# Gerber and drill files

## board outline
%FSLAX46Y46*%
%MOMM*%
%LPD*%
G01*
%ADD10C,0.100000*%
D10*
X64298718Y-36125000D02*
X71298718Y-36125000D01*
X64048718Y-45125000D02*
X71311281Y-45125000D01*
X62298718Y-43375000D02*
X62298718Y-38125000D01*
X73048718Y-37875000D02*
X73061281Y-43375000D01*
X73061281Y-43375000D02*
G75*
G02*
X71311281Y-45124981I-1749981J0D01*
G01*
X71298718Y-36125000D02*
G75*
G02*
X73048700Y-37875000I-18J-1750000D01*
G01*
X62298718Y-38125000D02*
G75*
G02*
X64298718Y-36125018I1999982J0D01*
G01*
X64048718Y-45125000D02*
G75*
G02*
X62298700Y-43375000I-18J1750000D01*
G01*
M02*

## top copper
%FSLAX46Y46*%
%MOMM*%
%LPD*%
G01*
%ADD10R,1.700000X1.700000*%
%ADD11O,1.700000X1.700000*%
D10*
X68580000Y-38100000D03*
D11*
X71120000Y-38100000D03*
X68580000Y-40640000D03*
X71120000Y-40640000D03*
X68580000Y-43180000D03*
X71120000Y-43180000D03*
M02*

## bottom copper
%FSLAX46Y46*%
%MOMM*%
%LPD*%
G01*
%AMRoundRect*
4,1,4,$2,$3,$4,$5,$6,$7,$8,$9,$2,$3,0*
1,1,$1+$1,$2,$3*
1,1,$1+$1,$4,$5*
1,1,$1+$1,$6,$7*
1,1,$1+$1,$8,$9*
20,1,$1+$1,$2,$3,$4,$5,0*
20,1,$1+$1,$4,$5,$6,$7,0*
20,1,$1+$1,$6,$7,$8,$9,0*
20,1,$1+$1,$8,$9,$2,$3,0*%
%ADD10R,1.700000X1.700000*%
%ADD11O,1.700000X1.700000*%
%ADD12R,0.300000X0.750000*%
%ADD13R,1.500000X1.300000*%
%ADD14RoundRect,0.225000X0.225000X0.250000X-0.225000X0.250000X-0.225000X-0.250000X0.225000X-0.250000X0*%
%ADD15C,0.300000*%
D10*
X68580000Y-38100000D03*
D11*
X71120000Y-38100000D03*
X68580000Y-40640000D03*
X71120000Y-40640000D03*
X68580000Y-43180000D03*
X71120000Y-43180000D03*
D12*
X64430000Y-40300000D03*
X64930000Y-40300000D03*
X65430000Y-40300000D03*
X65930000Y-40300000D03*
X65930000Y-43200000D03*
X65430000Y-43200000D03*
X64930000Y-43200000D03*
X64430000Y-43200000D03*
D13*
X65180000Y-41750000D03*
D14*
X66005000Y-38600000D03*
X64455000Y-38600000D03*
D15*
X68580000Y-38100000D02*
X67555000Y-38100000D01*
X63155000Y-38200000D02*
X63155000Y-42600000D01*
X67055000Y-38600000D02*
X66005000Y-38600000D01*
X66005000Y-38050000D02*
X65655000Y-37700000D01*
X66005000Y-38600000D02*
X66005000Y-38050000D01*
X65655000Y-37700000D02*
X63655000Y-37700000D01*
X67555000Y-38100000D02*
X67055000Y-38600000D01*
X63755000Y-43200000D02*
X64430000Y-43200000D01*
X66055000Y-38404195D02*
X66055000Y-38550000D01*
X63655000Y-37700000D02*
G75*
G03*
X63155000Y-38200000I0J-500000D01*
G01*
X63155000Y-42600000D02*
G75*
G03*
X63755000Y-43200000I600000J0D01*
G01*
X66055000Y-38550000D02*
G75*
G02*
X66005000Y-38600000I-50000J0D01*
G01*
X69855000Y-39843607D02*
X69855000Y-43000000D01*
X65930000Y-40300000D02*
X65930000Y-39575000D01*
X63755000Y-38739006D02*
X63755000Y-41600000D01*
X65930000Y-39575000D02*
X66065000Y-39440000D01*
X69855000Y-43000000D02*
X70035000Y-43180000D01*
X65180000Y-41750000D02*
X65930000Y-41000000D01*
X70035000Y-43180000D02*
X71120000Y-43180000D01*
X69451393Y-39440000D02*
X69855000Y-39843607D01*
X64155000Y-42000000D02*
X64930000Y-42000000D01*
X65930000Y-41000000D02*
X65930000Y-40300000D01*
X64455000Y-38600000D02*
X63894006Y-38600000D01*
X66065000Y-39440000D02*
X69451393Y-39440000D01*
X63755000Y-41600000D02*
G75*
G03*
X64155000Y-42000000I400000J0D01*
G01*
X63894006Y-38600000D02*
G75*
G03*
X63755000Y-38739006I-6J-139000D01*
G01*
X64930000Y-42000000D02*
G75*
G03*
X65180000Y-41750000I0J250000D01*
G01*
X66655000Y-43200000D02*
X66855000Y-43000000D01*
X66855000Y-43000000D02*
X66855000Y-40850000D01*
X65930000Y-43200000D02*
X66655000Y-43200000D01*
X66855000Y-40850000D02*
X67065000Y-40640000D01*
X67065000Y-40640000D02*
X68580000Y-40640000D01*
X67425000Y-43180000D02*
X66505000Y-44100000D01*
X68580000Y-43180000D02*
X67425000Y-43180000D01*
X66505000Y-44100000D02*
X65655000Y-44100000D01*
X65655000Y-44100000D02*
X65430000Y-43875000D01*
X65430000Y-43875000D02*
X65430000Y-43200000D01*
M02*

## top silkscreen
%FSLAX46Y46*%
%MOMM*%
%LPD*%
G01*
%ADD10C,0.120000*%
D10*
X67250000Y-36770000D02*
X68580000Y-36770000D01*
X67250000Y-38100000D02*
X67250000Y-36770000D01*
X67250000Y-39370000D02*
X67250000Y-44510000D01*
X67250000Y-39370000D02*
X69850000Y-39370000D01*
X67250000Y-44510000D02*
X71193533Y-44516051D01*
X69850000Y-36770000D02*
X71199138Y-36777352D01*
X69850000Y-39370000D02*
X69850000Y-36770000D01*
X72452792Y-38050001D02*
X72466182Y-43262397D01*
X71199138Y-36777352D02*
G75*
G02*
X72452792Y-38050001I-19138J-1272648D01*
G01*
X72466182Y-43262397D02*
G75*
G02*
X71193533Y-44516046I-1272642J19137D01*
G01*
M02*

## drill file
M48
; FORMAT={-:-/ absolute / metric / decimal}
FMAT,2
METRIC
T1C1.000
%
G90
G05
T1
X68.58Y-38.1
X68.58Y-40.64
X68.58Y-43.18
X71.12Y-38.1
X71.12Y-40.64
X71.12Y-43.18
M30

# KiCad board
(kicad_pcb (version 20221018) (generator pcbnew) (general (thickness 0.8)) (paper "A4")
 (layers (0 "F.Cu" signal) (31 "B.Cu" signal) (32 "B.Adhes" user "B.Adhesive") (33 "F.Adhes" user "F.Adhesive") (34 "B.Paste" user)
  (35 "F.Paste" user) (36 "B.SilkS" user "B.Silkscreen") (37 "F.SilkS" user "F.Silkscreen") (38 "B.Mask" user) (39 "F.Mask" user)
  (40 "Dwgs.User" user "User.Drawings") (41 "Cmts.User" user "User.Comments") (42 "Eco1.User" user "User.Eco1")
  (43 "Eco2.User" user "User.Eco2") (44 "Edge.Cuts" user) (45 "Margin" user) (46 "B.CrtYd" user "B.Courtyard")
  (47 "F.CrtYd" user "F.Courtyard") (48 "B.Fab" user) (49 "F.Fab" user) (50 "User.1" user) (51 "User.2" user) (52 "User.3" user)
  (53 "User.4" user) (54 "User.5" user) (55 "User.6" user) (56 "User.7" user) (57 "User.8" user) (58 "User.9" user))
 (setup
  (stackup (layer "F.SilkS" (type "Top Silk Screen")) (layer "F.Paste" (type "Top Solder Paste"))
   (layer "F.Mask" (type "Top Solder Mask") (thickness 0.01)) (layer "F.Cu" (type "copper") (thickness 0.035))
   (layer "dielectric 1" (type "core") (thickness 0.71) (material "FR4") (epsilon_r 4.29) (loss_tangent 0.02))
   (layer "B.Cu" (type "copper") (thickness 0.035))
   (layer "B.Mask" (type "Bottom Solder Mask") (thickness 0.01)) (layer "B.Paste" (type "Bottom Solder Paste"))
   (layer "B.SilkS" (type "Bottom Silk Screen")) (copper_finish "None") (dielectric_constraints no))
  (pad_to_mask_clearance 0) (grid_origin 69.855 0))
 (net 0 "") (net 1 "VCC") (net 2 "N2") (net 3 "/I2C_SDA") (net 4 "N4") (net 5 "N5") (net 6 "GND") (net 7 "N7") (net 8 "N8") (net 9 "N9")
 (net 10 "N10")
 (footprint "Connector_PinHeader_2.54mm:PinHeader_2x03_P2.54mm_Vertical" (layer "F.Cu") (at 68.58 38.1)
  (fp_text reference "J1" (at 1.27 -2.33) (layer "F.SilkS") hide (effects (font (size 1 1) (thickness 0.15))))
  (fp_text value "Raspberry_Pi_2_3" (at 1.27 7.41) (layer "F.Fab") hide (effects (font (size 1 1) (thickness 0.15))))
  (fp_line (start -1.33 -1.33) (end 0 -1.33) (stroke (width 0.12) (type solid)) (layer "F.SilkS"))
  (fp_line (start -1.33 0) (end -1.33 -1.33) (stroke (width 0.12) (type solid)) (layer "F.SilkS"))
  (fp_line (start -1.33 1.27) (end -1.33 6.41) (stroke (width 0.12) (type solid)) (layer "F.SilkS"))
  (fp_line (start -1.33 1.27) (end 1.27 1.27) (stroke (width 0.12) (type solid)) (layer "F.SilkS"))
  (fp_line (start -1.33 6.41) (end 2.613533 6.416051) (stroke (width 0.12) (type solid)) (layer "F.SilkS"))
  (fp_line (start 1.27 -1.33) (end 2.619138 -1.322648) (stroke (width 0.12) (type solid)) (layer "F.SilkS"))
  (fp_line (start 1.27 1.27) (end 1.27 -1.33) (stroke (width 0.12) (type solid)) (layer "F.SilkS"))
  (fp_line (start 3.872792 -0.049999) (end 3.886182 5.162397) (stroke (width 0.12) (type solid)) (layer "F.SilkS"))
  (fp_arc (start 2.619138 -1.322648) (mid 3.506741 -0.943207) (end 3.872792 -0.049999) (stroke (width 0.12) (type default))
   (layer "F.SilkS"))
  (fp_arc (start 3.886182 5.162397) (mid 3.506742 6.050002) (end 2.613533 6.416051) (stroke (width 0.12) (type default)) (layer "F.SilkS"))
  (pad "1" thru_hole rect (at 0 0) (size 1.7 1.7) (drill 1) (layers "*.Cu" "*.Mask") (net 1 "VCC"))
  (pad "2" thru_hole oval (at 2.54 0) (size 1.7 1.7) (drill 1) (layers "*.Cu" "*.Mask") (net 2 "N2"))
  (pad "3" thru_hole oval (at 0 2.54) (size 1.7 1.7) (drill 1) (layers "*.Cu" "*.Mask") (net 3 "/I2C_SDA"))
  (pad "4" thru_hole oval (at 2.54 2.54) (size 1.7 1.7) (drill 1) (layers "*.Cu" "*.Mask") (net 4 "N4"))
  (pad "5" thru_hole oval (at 0 5.08) (size 1.7 1.7) (drill 1) (layers "*.Cu" "*.Mask") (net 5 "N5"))
  (pad "6" thru_hole oval (at 2.54 5.08) (size 1.7 1.7) (drill 1) (layers "*.Cu" "*.Mask") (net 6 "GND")))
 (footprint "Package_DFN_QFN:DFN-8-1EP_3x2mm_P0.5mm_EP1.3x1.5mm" (layer "B.Cu") (at 65.18 41.75 -90)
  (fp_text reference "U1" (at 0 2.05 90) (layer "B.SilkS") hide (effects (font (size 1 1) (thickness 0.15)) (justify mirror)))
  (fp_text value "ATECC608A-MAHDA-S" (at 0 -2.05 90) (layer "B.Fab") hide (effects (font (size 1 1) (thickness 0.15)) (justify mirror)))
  (pad "" smd rect (at -0.325 -0.375 270) (size 0.5 0.6) (layers "B.Paste"))
  (pad "" smd rect (at -0.325 0.375 270) (size 0.5 0.6) (layers "B.Paste"))
  (pad "" smd rect (at 0.325 -0.375 270) (size 0.5 0.6) (layers "B.Paste"))
  (pad "" smd rect (at 0.325 0.375 270) (size 0.5 0.6) (layers "B.Paste"))
  (pad "1" smd rect (at -1.45 0.75 270) (size 0.75 0.3) (layers "B.Cu" "B.Paste" "B.Mask") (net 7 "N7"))
  (pad "2" smd rect (at -1.45 0.25 270) (size 0.75 0.3) (layers "B.Cu" "B.Paste" "B.Mask") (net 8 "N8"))
  (pad "3" smd rect (at -1.45 -0.25 270) (size 0.75 0.3) (layers "B.Cu" "B.Paste" "B.Mask") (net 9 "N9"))
  (pad "4" smd rect (at -1.45 -0.75 270) (size 0.75 0.3) (layers "B.Cu" "B.Paste" "B.Mask") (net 6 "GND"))
  (pad "5" smd rect (at 1.45 -0.75 270) (size 0.75 0.3) (layers "B.Cu" "B.Paste" "B.Mask") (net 3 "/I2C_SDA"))
  (pad "6" smd rect (at 1.45 -0.25 270) (size 0.75 0.3) (layers "B.Cu" "B.Paste" "B.Mask") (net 5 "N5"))
  (pad "7" smd rect (at 1.45 0.25 270) (size 0.75 0.3) (layers "B.Cu" "B.Paste" "B.Mask") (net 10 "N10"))
  (pad "8" smd rect (at 1.45 0.75 270) (size 0.75 0.3) (layers "B.Cu" "B.Paste" "B.Mask") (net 1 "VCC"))
  (pad "9" smd rect (at 0 0 270) (size 1.3 1.5) (layers "B.Cu" "B.Mask") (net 6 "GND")))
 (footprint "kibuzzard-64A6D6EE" (layer "B.Cu") (at 64.815 37 180)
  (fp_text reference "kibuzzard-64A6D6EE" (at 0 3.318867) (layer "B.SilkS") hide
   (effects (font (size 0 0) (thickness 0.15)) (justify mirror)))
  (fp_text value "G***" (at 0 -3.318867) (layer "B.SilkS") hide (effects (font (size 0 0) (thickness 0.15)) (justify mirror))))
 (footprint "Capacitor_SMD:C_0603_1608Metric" (layer "B.Cu") (at 65.23 38.6 180)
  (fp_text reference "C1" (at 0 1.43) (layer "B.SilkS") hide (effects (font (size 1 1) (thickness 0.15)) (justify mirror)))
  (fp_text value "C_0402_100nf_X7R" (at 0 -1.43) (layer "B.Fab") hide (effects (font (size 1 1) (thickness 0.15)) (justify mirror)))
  (pad "1" smd roundrect (at -0.775 0 180) (size 0.9 0.95) (layers "B.Cu" "B.Paste" "B.Mask") (roundrect_rratio 0.25) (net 1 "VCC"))
  (pad "2" smd roundrect (at 0.775 0 180) (size 0.9 0.95) (layers "B.Cu" "B.Paste" "B.Mask") (roundrect_rratio 0.25) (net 6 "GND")))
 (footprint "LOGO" (layer "B.Cu") (at 66.655 37)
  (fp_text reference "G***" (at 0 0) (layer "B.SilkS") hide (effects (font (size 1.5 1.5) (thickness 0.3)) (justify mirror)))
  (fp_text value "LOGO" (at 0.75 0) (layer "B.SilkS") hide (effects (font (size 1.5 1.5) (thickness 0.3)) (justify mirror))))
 (gr_line (start 64.298718 36.125) (end 71.298718 36.125) (stroke (width 0.1) (type default)) (layer "Edge.Cuts"))
 (gr_line (start 64.048718 45.125) (end 71.311281 45.125) (stroke (width 0.1) (type default)) (layer "Edge.Cuts"))
 (gr_line (start 62.298718 43.375) (end 62.298718 38.125) (stroke (width 0.1) (type default)) (layer "Edge.Cuts"))
 (gr_line (start 73.048718 37.875) (end 73.061281 43.375) (stroke (width 0.1) (type default)) (layer "Edge.Cuts"))
 (gr_arc (start 73.061281 43.375) (mid 72.548716 44.612424) (end 71.311281 45.125) (stroke (width 0.1) (type default)) (layer "Edge.Cuts"))
 (gr_arc (start 71.298718 36.125) (mid 72.536155 36.637563) (end 73.048718 37.875) (stroke (width 0.1) (type default)) (layer "Edge.Cuts"))
 (gr_arc (start 62.298718 38.125) (mid 62.884504 36.710786) (end 64.298718 36.125) (stroke (width 0.1) (type default)) (layer "Edge.Cuts"))
 (gr_arc (start 64.048718 45.125) (mid 62.811281 44.612437) (end 62.298718 43.375) (stroke (width 0.1) (type default)) (layer "Edge.Cuts"))
 (segment (start 68.58 38.1) (end 67.555 38.1) (width 0.3) (layer "B.Cu") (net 1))
 (segment (start 63.155 38.2) (end 63.155 42.6) (width 0.3) (layer "B.Cu") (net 1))
 (segment (start 67.055 38.6) (end 66.005 38.6) (width 0.3) (layer "B.Cu") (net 1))
 (segment (start 66.005 38.05) (end 65.655 37.7) (width 0.3) (layer "B.Cu") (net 1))
 (segment (start 66.005 38.6) (end 66.005 38.05) (width 0.3) (layer "B.Cu") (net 1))
 (segment (start 65.655 37.7) (end 63.655 37.7) (width 0.3) (layer "B.Cu") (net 1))
 (segment (start 67.555 38.1) (end 67.055 38.6) (width 0.3) (layer "B.Cu") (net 1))
 (segment (start 63.755 43.2) (end 64.43 43.2) (width 0.3) (layer "B.Cu") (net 1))
 (segment (start 66.055 38.404195) (end 66.055 38.55) (width 0.3) (layer "B.Cu") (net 1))
 (arc (start 63.655 37.7) (mid 63.301447 37.846447) (end 63.155 38.2) (width 0.3) (layer "B.Cu") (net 1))
 (arc (start 63.155 42.6) (mid 63.330736 43.024264) (end 63.755 43.2) (width 0.3) (layer "B.Cu") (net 1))
 (arc (start 66.055 38.55) (mid 66.040355 38.585355) (end 66.005 38.6) (width 0.3) (layer "B.Cu") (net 1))
 (segment (start 69.855 39.843607) (end 69.855 43) (width 0.3) (layer "B.Cu") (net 6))
 (segment (start 65.93 40.3) (end 65.93 39.575) (width 0.3) (layer "B.Cu") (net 6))
 (segment (start 63.755 38.739006) (end 63.755 41.6) (width 0.3) (layer "B.Cu") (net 6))
 (segment (start 65.93 39.575) (end 66.065 39.44) (width 0.3) (layer "B.Cu") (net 6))
 (segment (start 69.855 43) (end 70.035 43.18) (width 0.3) (layer "B.Cu") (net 6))
 (segment (start 65.18 41.75) (end 65.93 41) (width 0.3) (layer "B.Cu") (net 6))
 (segment (start 70.035 43.18) (end 71.12 43.18) (width 0.3) (layer "B.Cu") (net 6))
 (segment (start 69.451393 39.44) (end 69.855 39.843607) (width 0.3) (layer "B.Cu") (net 6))
 (segment (start 64.155 42) (end 64.93 42) (width 0.3) (layer "B.Cu") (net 6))
 (segment (start 65.93 41) (end 65.93 40.3) (width 0.3) (layer "B.Cu") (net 6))
 (segment (start 64.455 38.6) (end 63.894006 38.6) (width 0.3) (layer "B.Cu") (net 6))
 (segment (start 66.065 39.44) (end 69.451393 39.44) (width 0.3) (layer "B.Cu") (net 6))
 (arc (start 63.755 41.6) (mid 63.872157 41.882843) (end 64.155 42) (width 0.3) (layer "B.Cu") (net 6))
 (arc (start 63.894006 38.6) (mid 63.795714 38.640714) (end 63.755 38.739006) (width 0.3) (layer "B.Cu") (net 6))
 (arc (start 64.93 42) (mid 65.106777 41.926777) (end 65.18 41.75) (width 0.3) (layer "B.Cu") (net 6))
 (segment (start 66.655 43.2) (end 66.855 43) (width 0.3) (layer "B.Cu") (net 3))
 (segment (start 66.855 43) (end 66.855 40.85) (width 0.3) (layer "B.Cu") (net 3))
 (segment (start 65.93 43.2) (end 66.655 43.2) (width 0.3) (layer "B.Cu") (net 3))
 (segment (start 66.855 40.85) (end 67.065 40.64) (width 0.3) (layer "B.Cu") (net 3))
 (segment (start 67.065 40.64) (end 68.58 40.64) (width 0.3) (layer "B.Cu") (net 3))
 (segment (start 67.425 43.18) (end 66.505 44.1) (width 0.3) (layer "B.Cu") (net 5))
 (segment (start 68.58 43.18) (end 67.425 43.18) (width 0.3) (layer "B.Cu") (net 5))
 (segment (start 66.505 44.1) (end 65.655 44.1) (width 0.3) (layer "B.Cu") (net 5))
 (segment (start 65.655 44.1) (end 65.43 43.875) (width 0.3) (layer "B.Cu") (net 5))
 (segment (start 65.43 43.875) (end 65.43 43.2) (width 0.3) (layer "B.Cu") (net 5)))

